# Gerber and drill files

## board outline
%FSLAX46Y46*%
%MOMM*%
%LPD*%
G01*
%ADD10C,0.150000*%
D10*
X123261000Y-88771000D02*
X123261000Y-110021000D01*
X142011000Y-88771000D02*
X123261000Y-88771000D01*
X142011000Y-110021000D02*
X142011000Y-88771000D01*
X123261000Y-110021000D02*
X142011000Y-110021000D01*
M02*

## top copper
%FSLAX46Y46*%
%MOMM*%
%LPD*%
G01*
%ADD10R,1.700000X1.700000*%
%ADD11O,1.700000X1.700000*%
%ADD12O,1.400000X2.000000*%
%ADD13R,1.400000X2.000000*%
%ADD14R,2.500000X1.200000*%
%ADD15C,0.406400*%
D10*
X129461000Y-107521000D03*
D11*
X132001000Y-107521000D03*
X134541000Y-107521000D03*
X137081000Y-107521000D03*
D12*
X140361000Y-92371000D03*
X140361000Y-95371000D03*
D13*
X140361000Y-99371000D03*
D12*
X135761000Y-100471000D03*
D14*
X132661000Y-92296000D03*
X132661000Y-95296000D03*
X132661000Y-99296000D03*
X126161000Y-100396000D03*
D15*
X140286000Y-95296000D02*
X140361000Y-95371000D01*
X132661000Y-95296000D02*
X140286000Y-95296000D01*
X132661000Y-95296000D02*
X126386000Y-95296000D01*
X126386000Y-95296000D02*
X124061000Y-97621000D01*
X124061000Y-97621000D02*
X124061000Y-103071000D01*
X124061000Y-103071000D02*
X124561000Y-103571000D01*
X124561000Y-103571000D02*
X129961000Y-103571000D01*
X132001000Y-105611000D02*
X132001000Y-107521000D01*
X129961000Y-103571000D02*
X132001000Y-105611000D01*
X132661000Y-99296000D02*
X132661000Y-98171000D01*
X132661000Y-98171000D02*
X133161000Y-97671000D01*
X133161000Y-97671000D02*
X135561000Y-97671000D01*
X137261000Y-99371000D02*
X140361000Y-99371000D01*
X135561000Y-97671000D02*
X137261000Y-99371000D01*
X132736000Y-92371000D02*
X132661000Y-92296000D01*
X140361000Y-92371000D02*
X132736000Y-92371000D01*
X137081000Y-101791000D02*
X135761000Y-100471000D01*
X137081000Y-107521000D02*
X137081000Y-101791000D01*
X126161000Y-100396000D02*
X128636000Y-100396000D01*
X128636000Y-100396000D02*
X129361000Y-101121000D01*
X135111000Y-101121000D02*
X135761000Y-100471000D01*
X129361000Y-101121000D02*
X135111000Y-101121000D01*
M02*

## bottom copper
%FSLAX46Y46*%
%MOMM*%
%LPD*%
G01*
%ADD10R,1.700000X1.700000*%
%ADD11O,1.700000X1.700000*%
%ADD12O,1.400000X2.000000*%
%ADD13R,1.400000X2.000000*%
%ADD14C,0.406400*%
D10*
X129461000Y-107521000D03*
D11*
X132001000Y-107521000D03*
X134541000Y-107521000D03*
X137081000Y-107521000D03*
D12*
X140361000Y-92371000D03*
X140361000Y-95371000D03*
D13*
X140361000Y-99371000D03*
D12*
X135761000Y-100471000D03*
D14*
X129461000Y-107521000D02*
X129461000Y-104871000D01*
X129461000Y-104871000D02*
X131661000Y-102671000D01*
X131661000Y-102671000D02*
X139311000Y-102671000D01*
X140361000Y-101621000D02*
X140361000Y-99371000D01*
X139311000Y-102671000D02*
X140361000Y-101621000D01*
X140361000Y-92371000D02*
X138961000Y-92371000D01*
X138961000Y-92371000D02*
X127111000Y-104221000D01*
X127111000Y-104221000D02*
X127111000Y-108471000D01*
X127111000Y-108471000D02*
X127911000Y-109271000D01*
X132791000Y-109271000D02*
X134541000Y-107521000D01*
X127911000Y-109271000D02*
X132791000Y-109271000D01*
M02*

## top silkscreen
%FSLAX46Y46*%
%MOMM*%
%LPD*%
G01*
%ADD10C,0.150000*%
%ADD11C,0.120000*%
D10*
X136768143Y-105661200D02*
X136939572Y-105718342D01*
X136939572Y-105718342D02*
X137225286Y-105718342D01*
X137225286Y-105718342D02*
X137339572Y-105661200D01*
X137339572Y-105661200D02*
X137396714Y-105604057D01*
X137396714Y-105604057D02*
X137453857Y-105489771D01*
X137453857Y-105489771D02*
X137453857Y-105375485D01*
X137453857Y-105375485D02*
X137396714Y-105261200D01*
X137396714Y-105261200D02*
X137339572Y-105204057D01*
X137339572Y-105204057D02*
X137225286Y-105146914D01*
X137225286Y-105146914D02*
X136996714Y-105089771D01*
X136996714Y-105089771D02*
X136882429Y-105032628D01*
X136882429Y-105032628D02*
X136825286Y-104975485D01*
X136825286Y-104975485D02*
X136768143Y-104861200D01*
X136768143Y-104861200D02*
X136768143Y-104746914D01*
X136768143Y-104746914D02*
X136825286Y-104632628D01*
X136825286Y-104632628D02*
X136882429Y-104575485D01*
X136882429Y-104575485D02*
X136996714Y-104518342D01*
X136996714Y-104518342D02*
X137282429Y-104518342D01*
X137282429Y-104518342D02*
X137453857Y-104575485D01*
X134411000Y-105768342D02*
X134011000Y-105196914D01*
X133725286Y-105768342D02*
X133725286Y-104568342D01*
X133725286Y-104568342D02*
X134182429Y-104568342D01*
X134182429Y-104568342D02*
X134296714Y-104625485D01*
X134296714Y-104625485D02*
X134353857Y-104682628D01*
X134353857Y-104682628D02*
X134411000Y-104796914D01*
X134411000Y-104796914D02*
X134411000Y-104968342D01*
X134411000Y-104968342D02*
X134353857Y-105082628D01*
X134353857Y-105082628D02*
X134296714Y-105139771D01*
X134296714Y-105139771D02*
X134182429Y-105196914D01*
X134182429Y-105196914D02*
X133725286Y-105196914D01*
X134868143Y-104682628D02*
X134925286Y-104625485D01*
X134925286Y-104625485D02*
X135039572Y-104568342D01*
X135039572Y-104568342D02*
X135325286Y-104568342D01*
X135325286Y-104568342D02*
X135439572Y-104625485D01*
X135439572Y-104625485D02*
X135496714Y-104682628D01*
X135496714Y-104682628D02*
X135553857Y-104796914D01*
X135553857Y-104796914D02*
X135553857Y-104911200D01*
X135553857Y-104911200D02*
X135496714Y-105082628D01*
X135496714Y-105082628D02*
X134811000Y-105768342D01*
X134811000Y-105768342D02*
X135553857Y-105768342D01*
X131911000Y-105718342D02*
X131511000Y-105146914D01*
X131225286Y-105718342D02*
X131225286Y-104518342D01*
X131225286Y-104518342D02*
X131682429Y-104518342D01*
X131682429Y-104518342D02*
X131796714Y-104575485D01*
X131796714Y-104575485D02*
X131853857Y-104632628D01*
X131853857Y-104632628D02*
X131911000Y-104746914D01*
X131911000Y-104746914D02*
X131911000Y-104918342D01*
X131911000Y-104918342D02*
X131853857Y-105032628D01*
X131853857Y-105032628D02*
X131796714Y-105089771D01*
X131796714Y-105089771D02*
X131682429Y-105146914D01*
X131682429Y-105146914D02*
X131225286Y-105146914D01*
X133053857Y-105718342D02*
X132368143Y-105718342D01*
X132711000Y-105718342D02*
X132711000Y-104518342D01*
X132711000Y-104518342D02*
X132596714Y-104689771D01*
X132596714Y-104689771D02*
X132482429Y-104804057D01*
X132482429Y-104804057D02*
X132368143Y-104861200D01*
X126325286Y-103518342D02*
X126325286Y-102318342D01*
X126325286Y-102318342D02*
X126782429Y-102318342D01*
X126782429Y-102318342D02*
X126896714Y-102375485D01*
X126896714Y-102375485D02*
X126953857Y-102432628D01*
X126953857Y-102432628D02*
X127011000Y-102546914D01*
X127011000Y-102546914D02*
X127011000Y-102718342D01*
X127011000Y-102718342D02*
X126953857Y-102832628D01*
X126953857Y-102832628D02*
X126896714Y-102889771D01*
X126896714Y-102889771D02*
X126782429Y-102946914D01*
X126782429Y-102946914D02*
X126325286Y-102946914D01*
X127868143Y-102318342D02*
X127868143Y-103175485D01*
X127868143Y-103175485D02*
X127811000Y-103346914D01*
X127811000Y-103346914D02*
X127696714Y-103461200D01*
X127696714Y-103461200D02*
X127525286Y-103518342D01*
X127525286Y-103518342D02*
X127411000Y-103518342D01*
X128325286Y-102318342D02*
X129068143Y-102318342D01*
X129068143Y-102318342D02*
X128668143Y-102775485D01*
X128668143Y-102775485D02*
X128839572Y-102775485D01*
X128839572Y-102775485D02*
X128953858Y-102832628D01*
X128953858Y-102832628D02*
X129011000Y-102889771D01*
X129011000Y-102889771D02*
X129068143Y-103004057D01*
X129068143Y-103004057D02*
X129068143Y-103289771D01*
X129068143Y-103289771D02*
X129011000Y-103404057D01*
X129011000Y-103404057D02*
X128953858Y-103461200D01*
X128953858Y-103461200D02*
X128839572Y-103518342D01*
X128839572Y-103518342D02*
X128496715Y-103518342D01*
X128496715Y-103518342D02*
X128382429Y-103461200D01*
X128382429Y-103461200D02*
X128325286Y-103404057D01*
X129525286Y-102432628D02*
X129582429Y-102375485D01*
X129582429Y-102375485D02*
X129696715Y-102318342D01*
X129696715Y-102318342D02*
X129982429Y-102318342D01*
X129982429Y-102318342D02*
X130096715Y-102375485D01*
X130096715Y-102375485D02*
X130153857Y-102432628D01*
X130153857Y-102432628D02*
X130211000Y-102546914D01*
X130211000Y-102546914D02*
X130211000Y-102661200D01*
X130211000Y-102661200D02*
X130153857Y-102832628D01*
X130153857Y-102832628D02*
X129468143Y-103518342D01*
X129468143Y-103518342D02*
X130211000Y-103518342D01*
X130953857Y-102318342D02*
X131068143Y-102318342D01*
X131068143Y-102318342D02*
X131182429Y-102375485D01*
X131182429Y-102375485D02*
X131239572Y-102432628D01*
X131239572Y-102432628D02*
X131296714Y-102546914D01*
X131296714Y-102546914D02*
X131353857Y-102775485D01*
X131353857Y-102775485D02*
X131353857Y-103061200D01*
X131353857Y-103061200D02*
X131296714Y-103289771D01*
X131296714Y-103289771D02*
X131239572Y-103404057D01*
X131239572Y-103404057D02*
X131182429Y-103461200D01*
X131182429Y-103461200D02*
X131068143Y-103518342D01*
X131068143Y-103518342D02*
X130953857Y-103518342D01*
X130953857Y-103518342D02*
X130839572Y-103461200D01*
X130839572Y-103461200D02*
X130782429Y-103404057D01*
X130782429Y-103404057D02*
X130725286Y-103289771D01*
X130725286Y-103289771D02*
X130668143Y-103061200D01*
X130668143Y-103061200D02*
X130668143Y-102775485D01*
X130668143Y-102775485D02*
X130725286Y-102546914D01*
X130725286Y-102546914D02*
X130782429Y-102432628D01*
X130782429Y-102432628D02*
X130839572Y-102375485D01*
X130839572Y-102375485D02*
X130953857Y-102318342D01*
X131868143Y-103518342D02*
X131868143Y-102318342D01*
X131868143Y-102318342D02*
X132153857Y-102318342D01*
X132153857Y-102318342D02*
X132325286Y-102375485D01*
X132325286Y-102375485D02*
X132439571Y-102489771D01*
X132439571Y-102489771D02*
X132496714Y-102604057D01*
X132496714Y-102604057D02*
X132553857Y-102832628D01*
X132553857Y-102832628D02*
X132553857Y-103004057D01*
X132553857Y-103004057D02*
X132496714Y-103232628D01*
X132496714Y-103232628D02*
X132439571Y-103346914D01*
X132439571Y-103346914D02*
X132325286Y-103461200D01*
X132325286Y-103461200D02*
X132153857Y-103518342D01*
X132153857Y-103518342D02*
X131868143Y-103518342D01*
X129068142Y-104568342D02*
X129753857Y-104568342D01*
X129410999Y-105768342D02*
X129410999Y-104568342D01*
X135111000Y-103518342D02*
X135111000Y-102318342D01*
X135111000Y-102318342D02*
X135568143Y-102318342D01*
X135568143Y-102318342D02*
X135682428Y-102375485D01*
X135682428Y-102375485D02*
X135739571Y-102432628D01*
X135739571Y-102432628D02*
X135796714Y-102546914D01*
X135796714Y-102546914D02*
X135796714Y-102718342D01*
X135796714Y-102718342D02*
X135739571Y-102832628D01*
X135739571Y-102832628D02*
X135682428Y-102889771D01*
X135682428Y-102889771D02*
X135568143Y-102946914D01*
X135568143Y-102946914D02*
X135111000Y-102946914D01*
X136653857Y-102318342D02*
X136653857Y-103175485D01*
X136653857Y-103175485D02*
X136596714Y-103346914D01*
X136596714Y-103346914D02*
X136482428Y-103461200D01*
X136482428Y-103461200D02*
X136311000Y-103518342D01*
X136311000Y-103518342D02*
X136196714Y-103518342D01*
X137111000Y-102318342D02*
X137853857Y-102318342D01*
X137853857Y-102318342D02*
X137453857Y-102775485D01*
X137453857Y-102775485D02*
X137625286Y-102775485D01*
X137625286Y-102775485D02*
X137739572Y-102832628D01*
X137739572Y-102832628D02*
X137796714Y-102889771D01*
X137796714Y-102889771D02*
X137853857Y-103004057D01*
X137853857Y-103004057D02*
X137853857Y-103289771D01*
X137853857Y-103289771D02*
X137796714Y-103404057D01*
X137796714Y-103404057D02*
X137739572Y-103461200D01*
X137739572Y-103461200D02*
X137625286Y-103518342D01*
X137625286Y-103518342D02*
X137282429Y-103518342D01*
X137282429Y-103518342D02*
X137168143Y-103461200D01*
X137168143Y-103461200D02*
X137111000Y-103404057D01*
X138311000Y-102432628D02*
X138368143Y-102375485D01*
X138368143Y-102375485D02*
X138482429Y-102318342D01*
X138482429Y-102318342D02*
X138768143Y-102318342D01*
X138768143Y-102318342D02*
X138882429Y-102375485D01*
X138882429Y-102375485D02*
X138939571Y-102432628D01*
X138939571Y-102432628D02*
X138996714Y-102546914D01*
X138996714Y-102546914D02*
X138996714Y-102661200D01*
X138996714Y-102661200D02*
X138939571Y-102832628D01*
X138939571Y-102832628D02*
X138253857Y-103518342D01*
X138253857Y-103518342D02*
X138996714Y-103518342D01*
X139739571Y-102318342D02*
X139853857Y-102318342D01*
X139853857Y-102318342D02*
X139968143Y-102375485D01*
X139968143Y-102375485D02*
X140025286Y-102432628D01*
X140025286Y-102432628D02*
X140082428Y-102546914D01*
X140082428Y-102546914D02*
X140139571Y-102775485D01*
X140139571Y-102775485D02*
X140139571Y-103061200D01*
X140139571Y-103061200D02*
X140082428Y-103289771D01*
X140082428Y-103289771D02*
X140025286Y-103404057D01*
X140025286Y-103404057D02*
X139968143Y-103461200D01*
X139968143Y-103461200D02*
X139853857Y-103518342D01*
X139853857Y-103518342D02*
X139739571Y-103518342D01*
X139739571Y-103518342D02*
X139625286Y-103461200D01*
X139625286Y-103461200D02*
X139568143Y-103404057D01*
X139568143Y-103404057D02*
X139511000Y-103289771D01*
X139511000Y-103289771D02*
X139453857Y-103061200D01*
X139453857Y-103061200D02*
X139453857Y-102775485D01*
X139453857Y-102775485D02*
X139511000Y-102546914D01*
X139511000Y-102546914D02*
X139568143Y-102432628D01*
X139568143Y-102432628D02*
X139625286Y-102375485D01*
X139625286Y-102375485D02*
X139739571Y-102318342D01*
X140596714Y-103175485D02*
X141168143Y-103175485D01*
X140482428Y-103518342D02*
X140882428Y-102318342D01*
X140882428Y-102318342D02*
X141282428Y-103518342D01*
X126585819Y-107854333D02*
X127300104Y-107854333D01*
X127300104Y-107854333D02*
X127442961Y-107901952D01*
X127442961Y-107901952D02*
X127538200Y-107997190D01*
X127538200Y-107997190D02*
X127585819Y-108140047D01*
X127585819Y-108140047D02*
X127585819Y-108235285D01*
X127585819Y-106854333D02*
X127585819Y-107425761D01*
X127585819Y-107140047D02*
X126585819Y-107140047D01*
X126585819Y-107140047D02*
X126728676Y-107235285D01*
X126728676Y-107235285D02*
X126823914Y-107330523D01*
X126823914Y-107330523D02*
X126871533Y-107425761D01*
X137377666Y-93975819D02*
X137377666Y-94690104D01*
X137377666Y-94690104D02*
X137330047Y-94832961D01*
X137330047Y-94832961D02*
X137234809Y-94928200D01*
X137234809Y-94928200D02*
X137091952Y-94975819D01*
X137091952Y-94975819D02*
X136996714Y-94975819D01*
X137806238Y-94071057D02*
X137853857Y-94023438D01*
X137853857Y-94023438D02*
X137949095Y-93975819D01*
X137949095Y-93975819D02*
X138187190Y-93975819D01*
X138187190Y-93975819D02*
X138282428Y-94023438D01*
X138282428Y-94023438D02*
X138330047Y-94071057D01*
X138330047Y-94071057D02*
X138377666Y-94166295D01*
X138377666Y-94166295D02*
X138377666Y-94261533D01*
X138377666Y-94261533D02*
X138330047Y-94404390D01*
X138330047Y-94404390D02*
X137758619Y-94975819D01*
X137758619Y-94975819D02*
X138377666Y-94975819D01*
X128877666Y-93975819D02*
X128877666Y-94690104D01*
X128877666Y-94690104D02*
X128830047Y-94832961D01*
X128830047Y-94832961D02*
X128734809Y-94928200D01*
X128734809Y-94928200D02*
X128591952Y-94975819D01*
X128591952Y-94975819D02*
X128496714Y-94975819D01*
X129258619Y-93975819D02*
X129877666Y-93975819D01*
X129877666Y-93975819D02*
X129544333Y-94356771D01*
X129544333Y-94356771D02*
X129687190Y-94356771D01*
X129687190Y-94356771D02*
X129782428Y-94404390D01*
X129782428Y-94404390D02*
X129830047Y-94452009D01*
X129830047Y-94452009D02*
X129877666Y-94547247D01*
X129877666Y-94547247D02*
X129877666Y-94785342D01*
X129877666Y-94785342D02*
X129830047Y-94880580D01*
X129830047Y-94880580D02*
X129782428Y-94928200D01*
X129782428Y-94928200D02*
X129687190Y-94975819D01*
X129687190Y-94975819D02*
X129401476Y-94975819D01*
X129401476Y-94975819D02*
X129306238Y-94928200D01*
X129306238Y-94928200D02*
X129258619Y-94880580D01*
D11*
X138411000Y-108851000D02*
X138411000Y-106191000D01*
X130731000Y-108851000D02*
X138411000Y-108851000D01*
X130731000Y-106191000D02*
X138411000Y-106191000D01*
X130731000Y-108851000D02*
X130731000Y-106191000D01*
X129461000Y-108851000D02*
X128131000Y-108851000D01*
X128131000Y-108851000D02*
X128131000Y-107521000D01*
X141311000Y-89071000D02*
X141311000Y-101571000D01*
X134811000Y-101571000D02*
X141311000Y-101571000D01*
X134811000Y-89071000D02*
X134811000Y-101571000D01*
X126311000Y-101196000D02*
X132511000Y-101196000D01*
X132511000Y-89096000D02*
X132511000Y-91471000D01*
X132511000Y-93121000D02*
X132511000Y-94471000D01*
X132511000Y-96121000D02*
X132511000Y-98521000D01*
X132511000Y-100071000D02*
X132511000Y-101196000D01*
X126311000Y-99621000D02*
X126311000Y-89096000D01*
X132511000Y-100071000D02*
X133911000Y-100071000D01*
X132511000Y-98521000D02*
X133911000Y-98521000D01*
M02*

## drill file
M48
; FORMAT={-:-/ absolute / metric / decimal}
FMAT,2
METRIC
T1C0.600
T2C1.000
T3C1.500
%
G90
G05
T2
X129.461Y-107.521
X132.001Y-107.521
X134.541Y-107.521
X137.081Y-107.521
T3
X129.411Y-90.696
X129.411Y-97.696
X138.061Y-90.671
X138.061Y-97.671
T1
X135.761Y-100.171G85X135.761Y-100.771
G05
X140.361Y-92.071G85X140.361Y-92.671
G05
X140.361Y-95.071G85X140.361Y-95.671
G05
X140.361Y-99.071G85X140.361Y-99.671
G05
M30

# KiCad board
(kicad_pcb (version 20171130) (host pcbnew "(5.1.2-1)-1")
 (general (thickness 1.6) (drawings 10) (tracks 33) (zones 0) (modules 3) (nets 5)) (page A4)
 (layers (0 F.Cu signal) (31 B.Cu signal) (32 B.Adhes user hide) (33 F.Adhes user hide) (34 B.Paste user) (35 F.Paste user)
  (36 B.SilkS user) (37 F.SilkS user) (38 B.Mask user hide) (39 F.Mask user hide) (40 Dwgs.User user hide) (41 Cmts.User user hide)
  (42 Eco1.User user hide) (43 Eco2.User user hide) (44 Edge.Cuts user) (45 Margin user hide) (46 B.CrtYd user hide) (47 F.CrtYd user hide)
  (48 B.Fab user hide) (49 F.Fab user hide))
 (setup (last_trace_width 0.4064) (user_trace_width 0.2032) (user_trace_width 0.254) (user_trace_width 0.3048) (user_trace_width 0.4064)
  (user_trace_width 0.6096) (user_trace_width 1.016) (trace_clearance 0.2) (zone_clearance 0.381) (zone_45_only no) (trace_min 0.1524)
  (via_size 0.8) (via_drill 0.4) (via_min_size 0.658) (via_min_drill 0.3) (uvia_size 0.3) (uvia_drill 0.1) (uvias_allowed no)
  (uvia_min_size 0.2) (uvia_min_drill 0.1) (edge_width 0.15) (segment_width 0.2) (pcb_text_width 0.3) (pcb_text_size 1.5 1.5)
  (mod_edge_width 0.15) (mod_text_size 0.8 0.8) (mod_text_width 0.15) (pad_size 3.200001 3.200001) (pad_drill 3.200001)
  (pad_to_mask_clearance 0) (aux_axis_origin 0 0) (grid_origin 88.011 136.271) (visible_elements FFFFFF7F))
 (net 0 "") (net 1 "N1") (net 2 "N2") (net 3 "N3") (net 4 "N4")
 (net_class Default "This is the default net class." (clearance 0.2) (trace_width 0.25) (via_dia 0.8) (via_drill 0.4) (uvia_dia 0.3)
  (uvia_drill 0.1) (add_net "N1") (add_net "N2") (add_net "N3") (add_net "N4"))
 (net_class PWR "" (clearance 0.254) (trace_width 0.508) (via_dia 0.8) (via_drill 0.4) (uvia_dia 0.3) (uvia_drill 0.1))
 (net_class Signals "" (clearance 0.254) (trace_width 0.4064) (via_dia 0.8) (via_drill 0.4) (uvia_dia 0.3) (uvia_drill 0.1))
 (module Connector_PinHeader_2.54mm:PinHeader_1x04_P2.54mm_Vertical (layer F.Cu) (at 129.461 107.521 90)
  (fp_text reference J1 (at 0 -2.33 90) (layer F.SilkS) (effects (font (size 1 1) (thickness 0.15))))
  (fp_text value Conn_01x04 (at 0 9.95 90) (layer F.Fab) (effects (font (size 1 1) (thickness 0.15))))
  (fp_line (start -1.33 8.95) (end 1.33 8.95) (layer F.SilkS) (width 0.12))
  (fp_line (start -1.33 1.27) (end -1.33 8.95) (layer F.SilkS) (width 0.12))
  (fp_line (start 1.33 1.27) (end 1.33 8.95) (layer F.SilkS) (width 0.12))
  (fp_line (start -1.33 1.27) (end 1.33 1.27) (layer F.SilkS) (width 0.12))
  (fp_line (start -1.33 0) (end -1.33 -1.33) (layer F.SilkS) (width 0.12))
  (fp_line (start -1.33 -1.33) (end 0 -1.33) (layer F.SilkS) (width 0.12))
  (pad 1 thru_hole rect (at 0 0 90) (size 1.7 1.7) (drill 1) (layers *.Cu *.Mask) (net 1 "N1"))
  (pad 2 thru_hole oval (at 0 2.54 90) (size 1.7 1.7) (drill 1) (layers *.Cu *.Mask) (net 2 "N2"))
  (pad 3 thru_hole oval (at 0 5.08 90) (size 1.7 1.7) (drill 1) (layers *.Cu *.Mask) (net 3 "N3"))
  (pad 4 thru_hole oval (at 0 7.62 90) (size 1.7 1.7) (drill 1) (layers *.Cu *.Mask) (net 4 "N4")))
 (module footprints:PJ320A (layer F.Cu) (at 135.311 99.371)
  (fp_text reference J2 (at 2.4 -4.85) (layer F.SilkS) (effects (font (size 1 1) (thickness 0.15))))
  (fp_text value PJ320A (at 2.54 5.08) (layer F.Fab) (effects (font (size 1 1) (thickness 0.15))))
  (fp_line (start 6 -10.3) (end 6 2.2) (layer F.SilkS) (width 0.12))
  (fp_line (start -0.5 2.2) (end 6 2.2) (layer F.SilkS) (width 0.12))
  (fp_line (start -0.5 -10.3) (end -0.5 2.2) (layer F.SilkS) (width 0.12))
  (pad "" np_thru_hole circle (at 2.75 -1.7 270) (size 1.5 1.5) (drill 1.5) (layers *.Cu *.Mask))
  (pad "" np_thru_hole circle (at 2.75 -8.7 270) (size 1.5 1.5) (drill 1.5) (layers *.Cu *.Mask))
  (pad R2 thru_hole oval (at 5.05 -7 270) (size 2 1.4) (drill oval 1.2 0.6) (layers *.Cu *.Mask) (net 3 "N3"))
  (pad R1 thru_hole oval (at 5.05 -4 270) (size 2 1.4) (drill oval 1.2 0.6) (layers *.Cu *.Mask) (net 2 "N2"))
  (pad T thru_hole rect (at 5.05 0 270) (size 2 1.4) (drill oval 1.2 0.6) (layers *.Cu *.Mask) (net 1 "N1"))
  (pad S thru_hole oval (at 0.45 1.1 270) (size 2 1.4) (drill oval 1.2 0.6) (layers *.Cu *.Mask) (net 4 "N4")))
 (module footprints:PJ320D (layer F.Cu) (at 129.411 95.471 270)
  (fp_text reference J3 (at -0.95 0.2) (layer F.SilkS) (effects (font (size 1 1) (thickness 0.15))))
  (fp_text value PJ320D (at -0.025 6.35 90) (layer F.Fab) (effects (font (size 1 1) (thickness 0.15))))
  (fp_line (start 5.725 3.1) (end 5.725 -3.1) (layer F.SilkS) (width 0.12))
  (fp_line (start -6.375 -3.1) (end -4 -3.1) (layer F.SilkS) (width 0.12))
  (fp_line (start -2.35 -3.1) (end -1 -3.1) (layer F.SilkS) (width 0.12))
  (fp_line (start 0.65 -3.1) (end 3.05 -3.1) (layer F.SilkS) (width 0.12))
  (fp_line (start 4.6 -3.1) (end 5.725 -3.1) (layer F.SilkS) (width 0.12))
  (fp_line (start 4.15 3.1) (end -6.375 3.1) (layer F.SilkS) (width 0.12))
  (fp_line (start 4.6 -3.1) (end 4.6 -4.5) (layer F.SilkS) (width 0.12))
  (fp_line (start 3.05 -3.1) (end 3.05 -4.5) (layer F.SilkS) (width 0.12))
  (pad "" np_thru_hole circle (at 2.225 0 270) (size 1.5 1.5) (drill 1.5) (layers *.Cu *.Mask))
  (pad "" np_thru_hole circle (at -4.775 0 270) (size 1.5 1.5) (drill 1.5) (layers *.Cu *.Mask))
  (pad R2 smd rect (at -3.175 -3.25 270) (size 1.2 2.5) (layers F.Cu F.Paste F.Mask) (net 3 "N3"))
  (pad R1 smd rect (at -0.175 -3.25 270) (size 1.2 2.5) (layers F.Cu F.Paste F.Mask) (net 2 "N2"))
  (pad T smd rect (at 3.825 -3.25 270) (size 1.2 2.5) (layers F.Cu F.Paste F.Mask) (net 1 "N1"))
  (pad S smd rect (at 4.925 3.25 270) (size 1.2 2.5) (layers F.Cu F.Paste F.Mask) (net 4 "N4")))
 (gr_line (start 123.261 88.771) (end 123.261 110.021) (layer Edge.Cuts) (width 0.15))
 (gr_line (start 142.011 88.771) (end 123.261 88.771) (layer Edge.Cuts) (width 0.15))
 (gr_line (start 142.011 110.021) (end 142.011 88.771) (layer Edge.Cuts) (width 0.15))
 (gr_line (start 123.261 110.021) (end 142.011 110.021) (layer Edge.Cuts) (width 0.15))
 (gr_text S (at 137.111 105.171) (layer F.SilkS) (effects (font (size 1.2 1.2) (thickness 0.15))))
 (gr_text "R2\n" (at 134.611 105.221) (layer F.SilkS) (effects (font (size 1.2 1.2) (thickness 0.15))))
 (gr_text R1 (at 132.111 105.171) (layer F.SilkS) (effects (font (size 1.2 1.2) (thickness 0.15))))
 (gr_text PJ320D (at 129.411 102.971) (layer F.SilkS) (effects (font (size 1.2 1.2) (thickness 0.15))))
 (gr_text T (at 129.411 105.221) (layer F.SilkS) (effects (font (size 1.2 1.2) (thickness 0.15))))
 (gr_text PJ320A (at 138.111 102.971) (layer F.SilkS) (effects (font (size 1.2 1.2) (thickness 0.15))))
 (segment (start 140.286 95.296) (end 140.361 95.371) (width 0.4064) (layer F.Cu) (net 2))
 (segment (start 132.661 95.296) (end 140.286 95.296) (width 0.4064) (layer F.Cu) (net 2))
 (segment (start 132.661 95.296) (end 126.386 95.296) (width 0.4064) (layer F.Cu) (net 2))
 (segment (start 126.386 95.296) (end 124.061 97.621) (width 0.4064) (layer F.Cu) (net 2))
 (segment (start 124.061 97.621) (end 124.061 103.071) (width 0.4064) (layer F.Cu) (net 2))
 (segment (start 124.061 103.071) (end 124.561 103.571) (width 0.4064) (layer F.Cu) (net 2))
 (segment (start 124.561 103.571) (end 129.961 103.571) (width 0.4064) (layer F.Cu) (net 2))
 (segment (start 132.001 105.611) (end 132.001 107.521) (width 0.4064) (layer F.Cu) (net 2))
 (segment (start 129.961 103.571) (end 132.001 105.611) (width 0.4064) (layer F.Cu) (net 2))
 (segment (start 132.661 99.296) (end 132.661 98.171) (width 0.4064) (layer F.Cu) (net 1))
 (segment (start 132.661 98.171) (end 133.161 97.671) (width 0.4064) (layer F.Cu) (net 1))
 (segment (start 133.161 97.671) (end 135.561 97.671) (width 0.4064) (layer F.Cu) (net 1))
 (segment (start 137.261 99.371) (end 140.361 99.371) (width 0.4064) (layer F.Cu) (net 1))
 (segment (start 135.561 97.671) (end 137.261 99.371) (width 0.4064) (layer F.Cu) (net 1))
 (segment (start 129.461 107.521) (end 129.461 104.871) (width 0.4064) (layer B.Cu) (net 1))
 (segment (start 129.461 104.871) (end 131.661 102.671) (width 0.4064) (layer B.Cu) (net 1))
 (segment (start 131.661 102.671) (end 139.311 102.671) (width 0.4064) (layer B.Cu) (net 1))
 (segment (start 140.361 101.621) (end 140.361 99.371) (width 0.4064) (layer B.Cu) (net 1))
 (segment (start 139.311 102.671) (end 140.361 101.621) (width 0.4064) (layer B.Cu) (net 1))
 (segment (start 132.736 92.371) (end 132.661 92.296) (width 0.4064) (layer F.Cu) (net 3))
 (segment (start 140.361 92.371) (end 132.736 92.371) (width 0.4064) (layer F.Cu) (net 3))
 (segment (start 140.361 92.371) (end 138.961 92.371) (width 0.4064) (layer B.Cu) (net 3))
 (segment (start 138.961 92.371) (end 127.111 104.221) (width 0.4064) (layer B.Cu) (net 3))
 (segment (start 127.111 104.221) (end 127.111 108.471) (width 0.4064) (layer B.Cu) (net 3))
 (segment (start 127.111 108.471) (end 127.911 109.271) (width 0.4064) (layer B.Cu) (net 3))
 (segment (start 132.791 109.271) (end 134.541 107.521) (width 0.4064) (layer B.Cu) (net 3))
 (segment (start 127.911 109.271) (end 132.791 109.271) (width 0.4064) (layer B.Cu) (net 3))
 (segment (start 137.081 101.791) (end 135.761 100.471) (width 0.4064) (layer F.Cu) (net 4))
 (segment (start 137.081 107.521) (end 137.081 101.791) (width 0.4064) (layer F.Cu) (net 4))
 (segment (start 126.161 100.396) (end 128.636 100.396) (width 0.4064) (layer F.Cu) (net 4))
 (segment (start 128.636 100.396) (end 129.361 101.121) (width 0.4064) (layer F.Cu) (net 4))
 (segment (start 135.111 101.121) (end 135.761 100.471) (width 0.4064) (layer F.Cu) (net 4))
 (segment (start 129.361 101.121) (end 135.111 101.121) (width 0.4064) (layer F.Cu) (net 4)))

